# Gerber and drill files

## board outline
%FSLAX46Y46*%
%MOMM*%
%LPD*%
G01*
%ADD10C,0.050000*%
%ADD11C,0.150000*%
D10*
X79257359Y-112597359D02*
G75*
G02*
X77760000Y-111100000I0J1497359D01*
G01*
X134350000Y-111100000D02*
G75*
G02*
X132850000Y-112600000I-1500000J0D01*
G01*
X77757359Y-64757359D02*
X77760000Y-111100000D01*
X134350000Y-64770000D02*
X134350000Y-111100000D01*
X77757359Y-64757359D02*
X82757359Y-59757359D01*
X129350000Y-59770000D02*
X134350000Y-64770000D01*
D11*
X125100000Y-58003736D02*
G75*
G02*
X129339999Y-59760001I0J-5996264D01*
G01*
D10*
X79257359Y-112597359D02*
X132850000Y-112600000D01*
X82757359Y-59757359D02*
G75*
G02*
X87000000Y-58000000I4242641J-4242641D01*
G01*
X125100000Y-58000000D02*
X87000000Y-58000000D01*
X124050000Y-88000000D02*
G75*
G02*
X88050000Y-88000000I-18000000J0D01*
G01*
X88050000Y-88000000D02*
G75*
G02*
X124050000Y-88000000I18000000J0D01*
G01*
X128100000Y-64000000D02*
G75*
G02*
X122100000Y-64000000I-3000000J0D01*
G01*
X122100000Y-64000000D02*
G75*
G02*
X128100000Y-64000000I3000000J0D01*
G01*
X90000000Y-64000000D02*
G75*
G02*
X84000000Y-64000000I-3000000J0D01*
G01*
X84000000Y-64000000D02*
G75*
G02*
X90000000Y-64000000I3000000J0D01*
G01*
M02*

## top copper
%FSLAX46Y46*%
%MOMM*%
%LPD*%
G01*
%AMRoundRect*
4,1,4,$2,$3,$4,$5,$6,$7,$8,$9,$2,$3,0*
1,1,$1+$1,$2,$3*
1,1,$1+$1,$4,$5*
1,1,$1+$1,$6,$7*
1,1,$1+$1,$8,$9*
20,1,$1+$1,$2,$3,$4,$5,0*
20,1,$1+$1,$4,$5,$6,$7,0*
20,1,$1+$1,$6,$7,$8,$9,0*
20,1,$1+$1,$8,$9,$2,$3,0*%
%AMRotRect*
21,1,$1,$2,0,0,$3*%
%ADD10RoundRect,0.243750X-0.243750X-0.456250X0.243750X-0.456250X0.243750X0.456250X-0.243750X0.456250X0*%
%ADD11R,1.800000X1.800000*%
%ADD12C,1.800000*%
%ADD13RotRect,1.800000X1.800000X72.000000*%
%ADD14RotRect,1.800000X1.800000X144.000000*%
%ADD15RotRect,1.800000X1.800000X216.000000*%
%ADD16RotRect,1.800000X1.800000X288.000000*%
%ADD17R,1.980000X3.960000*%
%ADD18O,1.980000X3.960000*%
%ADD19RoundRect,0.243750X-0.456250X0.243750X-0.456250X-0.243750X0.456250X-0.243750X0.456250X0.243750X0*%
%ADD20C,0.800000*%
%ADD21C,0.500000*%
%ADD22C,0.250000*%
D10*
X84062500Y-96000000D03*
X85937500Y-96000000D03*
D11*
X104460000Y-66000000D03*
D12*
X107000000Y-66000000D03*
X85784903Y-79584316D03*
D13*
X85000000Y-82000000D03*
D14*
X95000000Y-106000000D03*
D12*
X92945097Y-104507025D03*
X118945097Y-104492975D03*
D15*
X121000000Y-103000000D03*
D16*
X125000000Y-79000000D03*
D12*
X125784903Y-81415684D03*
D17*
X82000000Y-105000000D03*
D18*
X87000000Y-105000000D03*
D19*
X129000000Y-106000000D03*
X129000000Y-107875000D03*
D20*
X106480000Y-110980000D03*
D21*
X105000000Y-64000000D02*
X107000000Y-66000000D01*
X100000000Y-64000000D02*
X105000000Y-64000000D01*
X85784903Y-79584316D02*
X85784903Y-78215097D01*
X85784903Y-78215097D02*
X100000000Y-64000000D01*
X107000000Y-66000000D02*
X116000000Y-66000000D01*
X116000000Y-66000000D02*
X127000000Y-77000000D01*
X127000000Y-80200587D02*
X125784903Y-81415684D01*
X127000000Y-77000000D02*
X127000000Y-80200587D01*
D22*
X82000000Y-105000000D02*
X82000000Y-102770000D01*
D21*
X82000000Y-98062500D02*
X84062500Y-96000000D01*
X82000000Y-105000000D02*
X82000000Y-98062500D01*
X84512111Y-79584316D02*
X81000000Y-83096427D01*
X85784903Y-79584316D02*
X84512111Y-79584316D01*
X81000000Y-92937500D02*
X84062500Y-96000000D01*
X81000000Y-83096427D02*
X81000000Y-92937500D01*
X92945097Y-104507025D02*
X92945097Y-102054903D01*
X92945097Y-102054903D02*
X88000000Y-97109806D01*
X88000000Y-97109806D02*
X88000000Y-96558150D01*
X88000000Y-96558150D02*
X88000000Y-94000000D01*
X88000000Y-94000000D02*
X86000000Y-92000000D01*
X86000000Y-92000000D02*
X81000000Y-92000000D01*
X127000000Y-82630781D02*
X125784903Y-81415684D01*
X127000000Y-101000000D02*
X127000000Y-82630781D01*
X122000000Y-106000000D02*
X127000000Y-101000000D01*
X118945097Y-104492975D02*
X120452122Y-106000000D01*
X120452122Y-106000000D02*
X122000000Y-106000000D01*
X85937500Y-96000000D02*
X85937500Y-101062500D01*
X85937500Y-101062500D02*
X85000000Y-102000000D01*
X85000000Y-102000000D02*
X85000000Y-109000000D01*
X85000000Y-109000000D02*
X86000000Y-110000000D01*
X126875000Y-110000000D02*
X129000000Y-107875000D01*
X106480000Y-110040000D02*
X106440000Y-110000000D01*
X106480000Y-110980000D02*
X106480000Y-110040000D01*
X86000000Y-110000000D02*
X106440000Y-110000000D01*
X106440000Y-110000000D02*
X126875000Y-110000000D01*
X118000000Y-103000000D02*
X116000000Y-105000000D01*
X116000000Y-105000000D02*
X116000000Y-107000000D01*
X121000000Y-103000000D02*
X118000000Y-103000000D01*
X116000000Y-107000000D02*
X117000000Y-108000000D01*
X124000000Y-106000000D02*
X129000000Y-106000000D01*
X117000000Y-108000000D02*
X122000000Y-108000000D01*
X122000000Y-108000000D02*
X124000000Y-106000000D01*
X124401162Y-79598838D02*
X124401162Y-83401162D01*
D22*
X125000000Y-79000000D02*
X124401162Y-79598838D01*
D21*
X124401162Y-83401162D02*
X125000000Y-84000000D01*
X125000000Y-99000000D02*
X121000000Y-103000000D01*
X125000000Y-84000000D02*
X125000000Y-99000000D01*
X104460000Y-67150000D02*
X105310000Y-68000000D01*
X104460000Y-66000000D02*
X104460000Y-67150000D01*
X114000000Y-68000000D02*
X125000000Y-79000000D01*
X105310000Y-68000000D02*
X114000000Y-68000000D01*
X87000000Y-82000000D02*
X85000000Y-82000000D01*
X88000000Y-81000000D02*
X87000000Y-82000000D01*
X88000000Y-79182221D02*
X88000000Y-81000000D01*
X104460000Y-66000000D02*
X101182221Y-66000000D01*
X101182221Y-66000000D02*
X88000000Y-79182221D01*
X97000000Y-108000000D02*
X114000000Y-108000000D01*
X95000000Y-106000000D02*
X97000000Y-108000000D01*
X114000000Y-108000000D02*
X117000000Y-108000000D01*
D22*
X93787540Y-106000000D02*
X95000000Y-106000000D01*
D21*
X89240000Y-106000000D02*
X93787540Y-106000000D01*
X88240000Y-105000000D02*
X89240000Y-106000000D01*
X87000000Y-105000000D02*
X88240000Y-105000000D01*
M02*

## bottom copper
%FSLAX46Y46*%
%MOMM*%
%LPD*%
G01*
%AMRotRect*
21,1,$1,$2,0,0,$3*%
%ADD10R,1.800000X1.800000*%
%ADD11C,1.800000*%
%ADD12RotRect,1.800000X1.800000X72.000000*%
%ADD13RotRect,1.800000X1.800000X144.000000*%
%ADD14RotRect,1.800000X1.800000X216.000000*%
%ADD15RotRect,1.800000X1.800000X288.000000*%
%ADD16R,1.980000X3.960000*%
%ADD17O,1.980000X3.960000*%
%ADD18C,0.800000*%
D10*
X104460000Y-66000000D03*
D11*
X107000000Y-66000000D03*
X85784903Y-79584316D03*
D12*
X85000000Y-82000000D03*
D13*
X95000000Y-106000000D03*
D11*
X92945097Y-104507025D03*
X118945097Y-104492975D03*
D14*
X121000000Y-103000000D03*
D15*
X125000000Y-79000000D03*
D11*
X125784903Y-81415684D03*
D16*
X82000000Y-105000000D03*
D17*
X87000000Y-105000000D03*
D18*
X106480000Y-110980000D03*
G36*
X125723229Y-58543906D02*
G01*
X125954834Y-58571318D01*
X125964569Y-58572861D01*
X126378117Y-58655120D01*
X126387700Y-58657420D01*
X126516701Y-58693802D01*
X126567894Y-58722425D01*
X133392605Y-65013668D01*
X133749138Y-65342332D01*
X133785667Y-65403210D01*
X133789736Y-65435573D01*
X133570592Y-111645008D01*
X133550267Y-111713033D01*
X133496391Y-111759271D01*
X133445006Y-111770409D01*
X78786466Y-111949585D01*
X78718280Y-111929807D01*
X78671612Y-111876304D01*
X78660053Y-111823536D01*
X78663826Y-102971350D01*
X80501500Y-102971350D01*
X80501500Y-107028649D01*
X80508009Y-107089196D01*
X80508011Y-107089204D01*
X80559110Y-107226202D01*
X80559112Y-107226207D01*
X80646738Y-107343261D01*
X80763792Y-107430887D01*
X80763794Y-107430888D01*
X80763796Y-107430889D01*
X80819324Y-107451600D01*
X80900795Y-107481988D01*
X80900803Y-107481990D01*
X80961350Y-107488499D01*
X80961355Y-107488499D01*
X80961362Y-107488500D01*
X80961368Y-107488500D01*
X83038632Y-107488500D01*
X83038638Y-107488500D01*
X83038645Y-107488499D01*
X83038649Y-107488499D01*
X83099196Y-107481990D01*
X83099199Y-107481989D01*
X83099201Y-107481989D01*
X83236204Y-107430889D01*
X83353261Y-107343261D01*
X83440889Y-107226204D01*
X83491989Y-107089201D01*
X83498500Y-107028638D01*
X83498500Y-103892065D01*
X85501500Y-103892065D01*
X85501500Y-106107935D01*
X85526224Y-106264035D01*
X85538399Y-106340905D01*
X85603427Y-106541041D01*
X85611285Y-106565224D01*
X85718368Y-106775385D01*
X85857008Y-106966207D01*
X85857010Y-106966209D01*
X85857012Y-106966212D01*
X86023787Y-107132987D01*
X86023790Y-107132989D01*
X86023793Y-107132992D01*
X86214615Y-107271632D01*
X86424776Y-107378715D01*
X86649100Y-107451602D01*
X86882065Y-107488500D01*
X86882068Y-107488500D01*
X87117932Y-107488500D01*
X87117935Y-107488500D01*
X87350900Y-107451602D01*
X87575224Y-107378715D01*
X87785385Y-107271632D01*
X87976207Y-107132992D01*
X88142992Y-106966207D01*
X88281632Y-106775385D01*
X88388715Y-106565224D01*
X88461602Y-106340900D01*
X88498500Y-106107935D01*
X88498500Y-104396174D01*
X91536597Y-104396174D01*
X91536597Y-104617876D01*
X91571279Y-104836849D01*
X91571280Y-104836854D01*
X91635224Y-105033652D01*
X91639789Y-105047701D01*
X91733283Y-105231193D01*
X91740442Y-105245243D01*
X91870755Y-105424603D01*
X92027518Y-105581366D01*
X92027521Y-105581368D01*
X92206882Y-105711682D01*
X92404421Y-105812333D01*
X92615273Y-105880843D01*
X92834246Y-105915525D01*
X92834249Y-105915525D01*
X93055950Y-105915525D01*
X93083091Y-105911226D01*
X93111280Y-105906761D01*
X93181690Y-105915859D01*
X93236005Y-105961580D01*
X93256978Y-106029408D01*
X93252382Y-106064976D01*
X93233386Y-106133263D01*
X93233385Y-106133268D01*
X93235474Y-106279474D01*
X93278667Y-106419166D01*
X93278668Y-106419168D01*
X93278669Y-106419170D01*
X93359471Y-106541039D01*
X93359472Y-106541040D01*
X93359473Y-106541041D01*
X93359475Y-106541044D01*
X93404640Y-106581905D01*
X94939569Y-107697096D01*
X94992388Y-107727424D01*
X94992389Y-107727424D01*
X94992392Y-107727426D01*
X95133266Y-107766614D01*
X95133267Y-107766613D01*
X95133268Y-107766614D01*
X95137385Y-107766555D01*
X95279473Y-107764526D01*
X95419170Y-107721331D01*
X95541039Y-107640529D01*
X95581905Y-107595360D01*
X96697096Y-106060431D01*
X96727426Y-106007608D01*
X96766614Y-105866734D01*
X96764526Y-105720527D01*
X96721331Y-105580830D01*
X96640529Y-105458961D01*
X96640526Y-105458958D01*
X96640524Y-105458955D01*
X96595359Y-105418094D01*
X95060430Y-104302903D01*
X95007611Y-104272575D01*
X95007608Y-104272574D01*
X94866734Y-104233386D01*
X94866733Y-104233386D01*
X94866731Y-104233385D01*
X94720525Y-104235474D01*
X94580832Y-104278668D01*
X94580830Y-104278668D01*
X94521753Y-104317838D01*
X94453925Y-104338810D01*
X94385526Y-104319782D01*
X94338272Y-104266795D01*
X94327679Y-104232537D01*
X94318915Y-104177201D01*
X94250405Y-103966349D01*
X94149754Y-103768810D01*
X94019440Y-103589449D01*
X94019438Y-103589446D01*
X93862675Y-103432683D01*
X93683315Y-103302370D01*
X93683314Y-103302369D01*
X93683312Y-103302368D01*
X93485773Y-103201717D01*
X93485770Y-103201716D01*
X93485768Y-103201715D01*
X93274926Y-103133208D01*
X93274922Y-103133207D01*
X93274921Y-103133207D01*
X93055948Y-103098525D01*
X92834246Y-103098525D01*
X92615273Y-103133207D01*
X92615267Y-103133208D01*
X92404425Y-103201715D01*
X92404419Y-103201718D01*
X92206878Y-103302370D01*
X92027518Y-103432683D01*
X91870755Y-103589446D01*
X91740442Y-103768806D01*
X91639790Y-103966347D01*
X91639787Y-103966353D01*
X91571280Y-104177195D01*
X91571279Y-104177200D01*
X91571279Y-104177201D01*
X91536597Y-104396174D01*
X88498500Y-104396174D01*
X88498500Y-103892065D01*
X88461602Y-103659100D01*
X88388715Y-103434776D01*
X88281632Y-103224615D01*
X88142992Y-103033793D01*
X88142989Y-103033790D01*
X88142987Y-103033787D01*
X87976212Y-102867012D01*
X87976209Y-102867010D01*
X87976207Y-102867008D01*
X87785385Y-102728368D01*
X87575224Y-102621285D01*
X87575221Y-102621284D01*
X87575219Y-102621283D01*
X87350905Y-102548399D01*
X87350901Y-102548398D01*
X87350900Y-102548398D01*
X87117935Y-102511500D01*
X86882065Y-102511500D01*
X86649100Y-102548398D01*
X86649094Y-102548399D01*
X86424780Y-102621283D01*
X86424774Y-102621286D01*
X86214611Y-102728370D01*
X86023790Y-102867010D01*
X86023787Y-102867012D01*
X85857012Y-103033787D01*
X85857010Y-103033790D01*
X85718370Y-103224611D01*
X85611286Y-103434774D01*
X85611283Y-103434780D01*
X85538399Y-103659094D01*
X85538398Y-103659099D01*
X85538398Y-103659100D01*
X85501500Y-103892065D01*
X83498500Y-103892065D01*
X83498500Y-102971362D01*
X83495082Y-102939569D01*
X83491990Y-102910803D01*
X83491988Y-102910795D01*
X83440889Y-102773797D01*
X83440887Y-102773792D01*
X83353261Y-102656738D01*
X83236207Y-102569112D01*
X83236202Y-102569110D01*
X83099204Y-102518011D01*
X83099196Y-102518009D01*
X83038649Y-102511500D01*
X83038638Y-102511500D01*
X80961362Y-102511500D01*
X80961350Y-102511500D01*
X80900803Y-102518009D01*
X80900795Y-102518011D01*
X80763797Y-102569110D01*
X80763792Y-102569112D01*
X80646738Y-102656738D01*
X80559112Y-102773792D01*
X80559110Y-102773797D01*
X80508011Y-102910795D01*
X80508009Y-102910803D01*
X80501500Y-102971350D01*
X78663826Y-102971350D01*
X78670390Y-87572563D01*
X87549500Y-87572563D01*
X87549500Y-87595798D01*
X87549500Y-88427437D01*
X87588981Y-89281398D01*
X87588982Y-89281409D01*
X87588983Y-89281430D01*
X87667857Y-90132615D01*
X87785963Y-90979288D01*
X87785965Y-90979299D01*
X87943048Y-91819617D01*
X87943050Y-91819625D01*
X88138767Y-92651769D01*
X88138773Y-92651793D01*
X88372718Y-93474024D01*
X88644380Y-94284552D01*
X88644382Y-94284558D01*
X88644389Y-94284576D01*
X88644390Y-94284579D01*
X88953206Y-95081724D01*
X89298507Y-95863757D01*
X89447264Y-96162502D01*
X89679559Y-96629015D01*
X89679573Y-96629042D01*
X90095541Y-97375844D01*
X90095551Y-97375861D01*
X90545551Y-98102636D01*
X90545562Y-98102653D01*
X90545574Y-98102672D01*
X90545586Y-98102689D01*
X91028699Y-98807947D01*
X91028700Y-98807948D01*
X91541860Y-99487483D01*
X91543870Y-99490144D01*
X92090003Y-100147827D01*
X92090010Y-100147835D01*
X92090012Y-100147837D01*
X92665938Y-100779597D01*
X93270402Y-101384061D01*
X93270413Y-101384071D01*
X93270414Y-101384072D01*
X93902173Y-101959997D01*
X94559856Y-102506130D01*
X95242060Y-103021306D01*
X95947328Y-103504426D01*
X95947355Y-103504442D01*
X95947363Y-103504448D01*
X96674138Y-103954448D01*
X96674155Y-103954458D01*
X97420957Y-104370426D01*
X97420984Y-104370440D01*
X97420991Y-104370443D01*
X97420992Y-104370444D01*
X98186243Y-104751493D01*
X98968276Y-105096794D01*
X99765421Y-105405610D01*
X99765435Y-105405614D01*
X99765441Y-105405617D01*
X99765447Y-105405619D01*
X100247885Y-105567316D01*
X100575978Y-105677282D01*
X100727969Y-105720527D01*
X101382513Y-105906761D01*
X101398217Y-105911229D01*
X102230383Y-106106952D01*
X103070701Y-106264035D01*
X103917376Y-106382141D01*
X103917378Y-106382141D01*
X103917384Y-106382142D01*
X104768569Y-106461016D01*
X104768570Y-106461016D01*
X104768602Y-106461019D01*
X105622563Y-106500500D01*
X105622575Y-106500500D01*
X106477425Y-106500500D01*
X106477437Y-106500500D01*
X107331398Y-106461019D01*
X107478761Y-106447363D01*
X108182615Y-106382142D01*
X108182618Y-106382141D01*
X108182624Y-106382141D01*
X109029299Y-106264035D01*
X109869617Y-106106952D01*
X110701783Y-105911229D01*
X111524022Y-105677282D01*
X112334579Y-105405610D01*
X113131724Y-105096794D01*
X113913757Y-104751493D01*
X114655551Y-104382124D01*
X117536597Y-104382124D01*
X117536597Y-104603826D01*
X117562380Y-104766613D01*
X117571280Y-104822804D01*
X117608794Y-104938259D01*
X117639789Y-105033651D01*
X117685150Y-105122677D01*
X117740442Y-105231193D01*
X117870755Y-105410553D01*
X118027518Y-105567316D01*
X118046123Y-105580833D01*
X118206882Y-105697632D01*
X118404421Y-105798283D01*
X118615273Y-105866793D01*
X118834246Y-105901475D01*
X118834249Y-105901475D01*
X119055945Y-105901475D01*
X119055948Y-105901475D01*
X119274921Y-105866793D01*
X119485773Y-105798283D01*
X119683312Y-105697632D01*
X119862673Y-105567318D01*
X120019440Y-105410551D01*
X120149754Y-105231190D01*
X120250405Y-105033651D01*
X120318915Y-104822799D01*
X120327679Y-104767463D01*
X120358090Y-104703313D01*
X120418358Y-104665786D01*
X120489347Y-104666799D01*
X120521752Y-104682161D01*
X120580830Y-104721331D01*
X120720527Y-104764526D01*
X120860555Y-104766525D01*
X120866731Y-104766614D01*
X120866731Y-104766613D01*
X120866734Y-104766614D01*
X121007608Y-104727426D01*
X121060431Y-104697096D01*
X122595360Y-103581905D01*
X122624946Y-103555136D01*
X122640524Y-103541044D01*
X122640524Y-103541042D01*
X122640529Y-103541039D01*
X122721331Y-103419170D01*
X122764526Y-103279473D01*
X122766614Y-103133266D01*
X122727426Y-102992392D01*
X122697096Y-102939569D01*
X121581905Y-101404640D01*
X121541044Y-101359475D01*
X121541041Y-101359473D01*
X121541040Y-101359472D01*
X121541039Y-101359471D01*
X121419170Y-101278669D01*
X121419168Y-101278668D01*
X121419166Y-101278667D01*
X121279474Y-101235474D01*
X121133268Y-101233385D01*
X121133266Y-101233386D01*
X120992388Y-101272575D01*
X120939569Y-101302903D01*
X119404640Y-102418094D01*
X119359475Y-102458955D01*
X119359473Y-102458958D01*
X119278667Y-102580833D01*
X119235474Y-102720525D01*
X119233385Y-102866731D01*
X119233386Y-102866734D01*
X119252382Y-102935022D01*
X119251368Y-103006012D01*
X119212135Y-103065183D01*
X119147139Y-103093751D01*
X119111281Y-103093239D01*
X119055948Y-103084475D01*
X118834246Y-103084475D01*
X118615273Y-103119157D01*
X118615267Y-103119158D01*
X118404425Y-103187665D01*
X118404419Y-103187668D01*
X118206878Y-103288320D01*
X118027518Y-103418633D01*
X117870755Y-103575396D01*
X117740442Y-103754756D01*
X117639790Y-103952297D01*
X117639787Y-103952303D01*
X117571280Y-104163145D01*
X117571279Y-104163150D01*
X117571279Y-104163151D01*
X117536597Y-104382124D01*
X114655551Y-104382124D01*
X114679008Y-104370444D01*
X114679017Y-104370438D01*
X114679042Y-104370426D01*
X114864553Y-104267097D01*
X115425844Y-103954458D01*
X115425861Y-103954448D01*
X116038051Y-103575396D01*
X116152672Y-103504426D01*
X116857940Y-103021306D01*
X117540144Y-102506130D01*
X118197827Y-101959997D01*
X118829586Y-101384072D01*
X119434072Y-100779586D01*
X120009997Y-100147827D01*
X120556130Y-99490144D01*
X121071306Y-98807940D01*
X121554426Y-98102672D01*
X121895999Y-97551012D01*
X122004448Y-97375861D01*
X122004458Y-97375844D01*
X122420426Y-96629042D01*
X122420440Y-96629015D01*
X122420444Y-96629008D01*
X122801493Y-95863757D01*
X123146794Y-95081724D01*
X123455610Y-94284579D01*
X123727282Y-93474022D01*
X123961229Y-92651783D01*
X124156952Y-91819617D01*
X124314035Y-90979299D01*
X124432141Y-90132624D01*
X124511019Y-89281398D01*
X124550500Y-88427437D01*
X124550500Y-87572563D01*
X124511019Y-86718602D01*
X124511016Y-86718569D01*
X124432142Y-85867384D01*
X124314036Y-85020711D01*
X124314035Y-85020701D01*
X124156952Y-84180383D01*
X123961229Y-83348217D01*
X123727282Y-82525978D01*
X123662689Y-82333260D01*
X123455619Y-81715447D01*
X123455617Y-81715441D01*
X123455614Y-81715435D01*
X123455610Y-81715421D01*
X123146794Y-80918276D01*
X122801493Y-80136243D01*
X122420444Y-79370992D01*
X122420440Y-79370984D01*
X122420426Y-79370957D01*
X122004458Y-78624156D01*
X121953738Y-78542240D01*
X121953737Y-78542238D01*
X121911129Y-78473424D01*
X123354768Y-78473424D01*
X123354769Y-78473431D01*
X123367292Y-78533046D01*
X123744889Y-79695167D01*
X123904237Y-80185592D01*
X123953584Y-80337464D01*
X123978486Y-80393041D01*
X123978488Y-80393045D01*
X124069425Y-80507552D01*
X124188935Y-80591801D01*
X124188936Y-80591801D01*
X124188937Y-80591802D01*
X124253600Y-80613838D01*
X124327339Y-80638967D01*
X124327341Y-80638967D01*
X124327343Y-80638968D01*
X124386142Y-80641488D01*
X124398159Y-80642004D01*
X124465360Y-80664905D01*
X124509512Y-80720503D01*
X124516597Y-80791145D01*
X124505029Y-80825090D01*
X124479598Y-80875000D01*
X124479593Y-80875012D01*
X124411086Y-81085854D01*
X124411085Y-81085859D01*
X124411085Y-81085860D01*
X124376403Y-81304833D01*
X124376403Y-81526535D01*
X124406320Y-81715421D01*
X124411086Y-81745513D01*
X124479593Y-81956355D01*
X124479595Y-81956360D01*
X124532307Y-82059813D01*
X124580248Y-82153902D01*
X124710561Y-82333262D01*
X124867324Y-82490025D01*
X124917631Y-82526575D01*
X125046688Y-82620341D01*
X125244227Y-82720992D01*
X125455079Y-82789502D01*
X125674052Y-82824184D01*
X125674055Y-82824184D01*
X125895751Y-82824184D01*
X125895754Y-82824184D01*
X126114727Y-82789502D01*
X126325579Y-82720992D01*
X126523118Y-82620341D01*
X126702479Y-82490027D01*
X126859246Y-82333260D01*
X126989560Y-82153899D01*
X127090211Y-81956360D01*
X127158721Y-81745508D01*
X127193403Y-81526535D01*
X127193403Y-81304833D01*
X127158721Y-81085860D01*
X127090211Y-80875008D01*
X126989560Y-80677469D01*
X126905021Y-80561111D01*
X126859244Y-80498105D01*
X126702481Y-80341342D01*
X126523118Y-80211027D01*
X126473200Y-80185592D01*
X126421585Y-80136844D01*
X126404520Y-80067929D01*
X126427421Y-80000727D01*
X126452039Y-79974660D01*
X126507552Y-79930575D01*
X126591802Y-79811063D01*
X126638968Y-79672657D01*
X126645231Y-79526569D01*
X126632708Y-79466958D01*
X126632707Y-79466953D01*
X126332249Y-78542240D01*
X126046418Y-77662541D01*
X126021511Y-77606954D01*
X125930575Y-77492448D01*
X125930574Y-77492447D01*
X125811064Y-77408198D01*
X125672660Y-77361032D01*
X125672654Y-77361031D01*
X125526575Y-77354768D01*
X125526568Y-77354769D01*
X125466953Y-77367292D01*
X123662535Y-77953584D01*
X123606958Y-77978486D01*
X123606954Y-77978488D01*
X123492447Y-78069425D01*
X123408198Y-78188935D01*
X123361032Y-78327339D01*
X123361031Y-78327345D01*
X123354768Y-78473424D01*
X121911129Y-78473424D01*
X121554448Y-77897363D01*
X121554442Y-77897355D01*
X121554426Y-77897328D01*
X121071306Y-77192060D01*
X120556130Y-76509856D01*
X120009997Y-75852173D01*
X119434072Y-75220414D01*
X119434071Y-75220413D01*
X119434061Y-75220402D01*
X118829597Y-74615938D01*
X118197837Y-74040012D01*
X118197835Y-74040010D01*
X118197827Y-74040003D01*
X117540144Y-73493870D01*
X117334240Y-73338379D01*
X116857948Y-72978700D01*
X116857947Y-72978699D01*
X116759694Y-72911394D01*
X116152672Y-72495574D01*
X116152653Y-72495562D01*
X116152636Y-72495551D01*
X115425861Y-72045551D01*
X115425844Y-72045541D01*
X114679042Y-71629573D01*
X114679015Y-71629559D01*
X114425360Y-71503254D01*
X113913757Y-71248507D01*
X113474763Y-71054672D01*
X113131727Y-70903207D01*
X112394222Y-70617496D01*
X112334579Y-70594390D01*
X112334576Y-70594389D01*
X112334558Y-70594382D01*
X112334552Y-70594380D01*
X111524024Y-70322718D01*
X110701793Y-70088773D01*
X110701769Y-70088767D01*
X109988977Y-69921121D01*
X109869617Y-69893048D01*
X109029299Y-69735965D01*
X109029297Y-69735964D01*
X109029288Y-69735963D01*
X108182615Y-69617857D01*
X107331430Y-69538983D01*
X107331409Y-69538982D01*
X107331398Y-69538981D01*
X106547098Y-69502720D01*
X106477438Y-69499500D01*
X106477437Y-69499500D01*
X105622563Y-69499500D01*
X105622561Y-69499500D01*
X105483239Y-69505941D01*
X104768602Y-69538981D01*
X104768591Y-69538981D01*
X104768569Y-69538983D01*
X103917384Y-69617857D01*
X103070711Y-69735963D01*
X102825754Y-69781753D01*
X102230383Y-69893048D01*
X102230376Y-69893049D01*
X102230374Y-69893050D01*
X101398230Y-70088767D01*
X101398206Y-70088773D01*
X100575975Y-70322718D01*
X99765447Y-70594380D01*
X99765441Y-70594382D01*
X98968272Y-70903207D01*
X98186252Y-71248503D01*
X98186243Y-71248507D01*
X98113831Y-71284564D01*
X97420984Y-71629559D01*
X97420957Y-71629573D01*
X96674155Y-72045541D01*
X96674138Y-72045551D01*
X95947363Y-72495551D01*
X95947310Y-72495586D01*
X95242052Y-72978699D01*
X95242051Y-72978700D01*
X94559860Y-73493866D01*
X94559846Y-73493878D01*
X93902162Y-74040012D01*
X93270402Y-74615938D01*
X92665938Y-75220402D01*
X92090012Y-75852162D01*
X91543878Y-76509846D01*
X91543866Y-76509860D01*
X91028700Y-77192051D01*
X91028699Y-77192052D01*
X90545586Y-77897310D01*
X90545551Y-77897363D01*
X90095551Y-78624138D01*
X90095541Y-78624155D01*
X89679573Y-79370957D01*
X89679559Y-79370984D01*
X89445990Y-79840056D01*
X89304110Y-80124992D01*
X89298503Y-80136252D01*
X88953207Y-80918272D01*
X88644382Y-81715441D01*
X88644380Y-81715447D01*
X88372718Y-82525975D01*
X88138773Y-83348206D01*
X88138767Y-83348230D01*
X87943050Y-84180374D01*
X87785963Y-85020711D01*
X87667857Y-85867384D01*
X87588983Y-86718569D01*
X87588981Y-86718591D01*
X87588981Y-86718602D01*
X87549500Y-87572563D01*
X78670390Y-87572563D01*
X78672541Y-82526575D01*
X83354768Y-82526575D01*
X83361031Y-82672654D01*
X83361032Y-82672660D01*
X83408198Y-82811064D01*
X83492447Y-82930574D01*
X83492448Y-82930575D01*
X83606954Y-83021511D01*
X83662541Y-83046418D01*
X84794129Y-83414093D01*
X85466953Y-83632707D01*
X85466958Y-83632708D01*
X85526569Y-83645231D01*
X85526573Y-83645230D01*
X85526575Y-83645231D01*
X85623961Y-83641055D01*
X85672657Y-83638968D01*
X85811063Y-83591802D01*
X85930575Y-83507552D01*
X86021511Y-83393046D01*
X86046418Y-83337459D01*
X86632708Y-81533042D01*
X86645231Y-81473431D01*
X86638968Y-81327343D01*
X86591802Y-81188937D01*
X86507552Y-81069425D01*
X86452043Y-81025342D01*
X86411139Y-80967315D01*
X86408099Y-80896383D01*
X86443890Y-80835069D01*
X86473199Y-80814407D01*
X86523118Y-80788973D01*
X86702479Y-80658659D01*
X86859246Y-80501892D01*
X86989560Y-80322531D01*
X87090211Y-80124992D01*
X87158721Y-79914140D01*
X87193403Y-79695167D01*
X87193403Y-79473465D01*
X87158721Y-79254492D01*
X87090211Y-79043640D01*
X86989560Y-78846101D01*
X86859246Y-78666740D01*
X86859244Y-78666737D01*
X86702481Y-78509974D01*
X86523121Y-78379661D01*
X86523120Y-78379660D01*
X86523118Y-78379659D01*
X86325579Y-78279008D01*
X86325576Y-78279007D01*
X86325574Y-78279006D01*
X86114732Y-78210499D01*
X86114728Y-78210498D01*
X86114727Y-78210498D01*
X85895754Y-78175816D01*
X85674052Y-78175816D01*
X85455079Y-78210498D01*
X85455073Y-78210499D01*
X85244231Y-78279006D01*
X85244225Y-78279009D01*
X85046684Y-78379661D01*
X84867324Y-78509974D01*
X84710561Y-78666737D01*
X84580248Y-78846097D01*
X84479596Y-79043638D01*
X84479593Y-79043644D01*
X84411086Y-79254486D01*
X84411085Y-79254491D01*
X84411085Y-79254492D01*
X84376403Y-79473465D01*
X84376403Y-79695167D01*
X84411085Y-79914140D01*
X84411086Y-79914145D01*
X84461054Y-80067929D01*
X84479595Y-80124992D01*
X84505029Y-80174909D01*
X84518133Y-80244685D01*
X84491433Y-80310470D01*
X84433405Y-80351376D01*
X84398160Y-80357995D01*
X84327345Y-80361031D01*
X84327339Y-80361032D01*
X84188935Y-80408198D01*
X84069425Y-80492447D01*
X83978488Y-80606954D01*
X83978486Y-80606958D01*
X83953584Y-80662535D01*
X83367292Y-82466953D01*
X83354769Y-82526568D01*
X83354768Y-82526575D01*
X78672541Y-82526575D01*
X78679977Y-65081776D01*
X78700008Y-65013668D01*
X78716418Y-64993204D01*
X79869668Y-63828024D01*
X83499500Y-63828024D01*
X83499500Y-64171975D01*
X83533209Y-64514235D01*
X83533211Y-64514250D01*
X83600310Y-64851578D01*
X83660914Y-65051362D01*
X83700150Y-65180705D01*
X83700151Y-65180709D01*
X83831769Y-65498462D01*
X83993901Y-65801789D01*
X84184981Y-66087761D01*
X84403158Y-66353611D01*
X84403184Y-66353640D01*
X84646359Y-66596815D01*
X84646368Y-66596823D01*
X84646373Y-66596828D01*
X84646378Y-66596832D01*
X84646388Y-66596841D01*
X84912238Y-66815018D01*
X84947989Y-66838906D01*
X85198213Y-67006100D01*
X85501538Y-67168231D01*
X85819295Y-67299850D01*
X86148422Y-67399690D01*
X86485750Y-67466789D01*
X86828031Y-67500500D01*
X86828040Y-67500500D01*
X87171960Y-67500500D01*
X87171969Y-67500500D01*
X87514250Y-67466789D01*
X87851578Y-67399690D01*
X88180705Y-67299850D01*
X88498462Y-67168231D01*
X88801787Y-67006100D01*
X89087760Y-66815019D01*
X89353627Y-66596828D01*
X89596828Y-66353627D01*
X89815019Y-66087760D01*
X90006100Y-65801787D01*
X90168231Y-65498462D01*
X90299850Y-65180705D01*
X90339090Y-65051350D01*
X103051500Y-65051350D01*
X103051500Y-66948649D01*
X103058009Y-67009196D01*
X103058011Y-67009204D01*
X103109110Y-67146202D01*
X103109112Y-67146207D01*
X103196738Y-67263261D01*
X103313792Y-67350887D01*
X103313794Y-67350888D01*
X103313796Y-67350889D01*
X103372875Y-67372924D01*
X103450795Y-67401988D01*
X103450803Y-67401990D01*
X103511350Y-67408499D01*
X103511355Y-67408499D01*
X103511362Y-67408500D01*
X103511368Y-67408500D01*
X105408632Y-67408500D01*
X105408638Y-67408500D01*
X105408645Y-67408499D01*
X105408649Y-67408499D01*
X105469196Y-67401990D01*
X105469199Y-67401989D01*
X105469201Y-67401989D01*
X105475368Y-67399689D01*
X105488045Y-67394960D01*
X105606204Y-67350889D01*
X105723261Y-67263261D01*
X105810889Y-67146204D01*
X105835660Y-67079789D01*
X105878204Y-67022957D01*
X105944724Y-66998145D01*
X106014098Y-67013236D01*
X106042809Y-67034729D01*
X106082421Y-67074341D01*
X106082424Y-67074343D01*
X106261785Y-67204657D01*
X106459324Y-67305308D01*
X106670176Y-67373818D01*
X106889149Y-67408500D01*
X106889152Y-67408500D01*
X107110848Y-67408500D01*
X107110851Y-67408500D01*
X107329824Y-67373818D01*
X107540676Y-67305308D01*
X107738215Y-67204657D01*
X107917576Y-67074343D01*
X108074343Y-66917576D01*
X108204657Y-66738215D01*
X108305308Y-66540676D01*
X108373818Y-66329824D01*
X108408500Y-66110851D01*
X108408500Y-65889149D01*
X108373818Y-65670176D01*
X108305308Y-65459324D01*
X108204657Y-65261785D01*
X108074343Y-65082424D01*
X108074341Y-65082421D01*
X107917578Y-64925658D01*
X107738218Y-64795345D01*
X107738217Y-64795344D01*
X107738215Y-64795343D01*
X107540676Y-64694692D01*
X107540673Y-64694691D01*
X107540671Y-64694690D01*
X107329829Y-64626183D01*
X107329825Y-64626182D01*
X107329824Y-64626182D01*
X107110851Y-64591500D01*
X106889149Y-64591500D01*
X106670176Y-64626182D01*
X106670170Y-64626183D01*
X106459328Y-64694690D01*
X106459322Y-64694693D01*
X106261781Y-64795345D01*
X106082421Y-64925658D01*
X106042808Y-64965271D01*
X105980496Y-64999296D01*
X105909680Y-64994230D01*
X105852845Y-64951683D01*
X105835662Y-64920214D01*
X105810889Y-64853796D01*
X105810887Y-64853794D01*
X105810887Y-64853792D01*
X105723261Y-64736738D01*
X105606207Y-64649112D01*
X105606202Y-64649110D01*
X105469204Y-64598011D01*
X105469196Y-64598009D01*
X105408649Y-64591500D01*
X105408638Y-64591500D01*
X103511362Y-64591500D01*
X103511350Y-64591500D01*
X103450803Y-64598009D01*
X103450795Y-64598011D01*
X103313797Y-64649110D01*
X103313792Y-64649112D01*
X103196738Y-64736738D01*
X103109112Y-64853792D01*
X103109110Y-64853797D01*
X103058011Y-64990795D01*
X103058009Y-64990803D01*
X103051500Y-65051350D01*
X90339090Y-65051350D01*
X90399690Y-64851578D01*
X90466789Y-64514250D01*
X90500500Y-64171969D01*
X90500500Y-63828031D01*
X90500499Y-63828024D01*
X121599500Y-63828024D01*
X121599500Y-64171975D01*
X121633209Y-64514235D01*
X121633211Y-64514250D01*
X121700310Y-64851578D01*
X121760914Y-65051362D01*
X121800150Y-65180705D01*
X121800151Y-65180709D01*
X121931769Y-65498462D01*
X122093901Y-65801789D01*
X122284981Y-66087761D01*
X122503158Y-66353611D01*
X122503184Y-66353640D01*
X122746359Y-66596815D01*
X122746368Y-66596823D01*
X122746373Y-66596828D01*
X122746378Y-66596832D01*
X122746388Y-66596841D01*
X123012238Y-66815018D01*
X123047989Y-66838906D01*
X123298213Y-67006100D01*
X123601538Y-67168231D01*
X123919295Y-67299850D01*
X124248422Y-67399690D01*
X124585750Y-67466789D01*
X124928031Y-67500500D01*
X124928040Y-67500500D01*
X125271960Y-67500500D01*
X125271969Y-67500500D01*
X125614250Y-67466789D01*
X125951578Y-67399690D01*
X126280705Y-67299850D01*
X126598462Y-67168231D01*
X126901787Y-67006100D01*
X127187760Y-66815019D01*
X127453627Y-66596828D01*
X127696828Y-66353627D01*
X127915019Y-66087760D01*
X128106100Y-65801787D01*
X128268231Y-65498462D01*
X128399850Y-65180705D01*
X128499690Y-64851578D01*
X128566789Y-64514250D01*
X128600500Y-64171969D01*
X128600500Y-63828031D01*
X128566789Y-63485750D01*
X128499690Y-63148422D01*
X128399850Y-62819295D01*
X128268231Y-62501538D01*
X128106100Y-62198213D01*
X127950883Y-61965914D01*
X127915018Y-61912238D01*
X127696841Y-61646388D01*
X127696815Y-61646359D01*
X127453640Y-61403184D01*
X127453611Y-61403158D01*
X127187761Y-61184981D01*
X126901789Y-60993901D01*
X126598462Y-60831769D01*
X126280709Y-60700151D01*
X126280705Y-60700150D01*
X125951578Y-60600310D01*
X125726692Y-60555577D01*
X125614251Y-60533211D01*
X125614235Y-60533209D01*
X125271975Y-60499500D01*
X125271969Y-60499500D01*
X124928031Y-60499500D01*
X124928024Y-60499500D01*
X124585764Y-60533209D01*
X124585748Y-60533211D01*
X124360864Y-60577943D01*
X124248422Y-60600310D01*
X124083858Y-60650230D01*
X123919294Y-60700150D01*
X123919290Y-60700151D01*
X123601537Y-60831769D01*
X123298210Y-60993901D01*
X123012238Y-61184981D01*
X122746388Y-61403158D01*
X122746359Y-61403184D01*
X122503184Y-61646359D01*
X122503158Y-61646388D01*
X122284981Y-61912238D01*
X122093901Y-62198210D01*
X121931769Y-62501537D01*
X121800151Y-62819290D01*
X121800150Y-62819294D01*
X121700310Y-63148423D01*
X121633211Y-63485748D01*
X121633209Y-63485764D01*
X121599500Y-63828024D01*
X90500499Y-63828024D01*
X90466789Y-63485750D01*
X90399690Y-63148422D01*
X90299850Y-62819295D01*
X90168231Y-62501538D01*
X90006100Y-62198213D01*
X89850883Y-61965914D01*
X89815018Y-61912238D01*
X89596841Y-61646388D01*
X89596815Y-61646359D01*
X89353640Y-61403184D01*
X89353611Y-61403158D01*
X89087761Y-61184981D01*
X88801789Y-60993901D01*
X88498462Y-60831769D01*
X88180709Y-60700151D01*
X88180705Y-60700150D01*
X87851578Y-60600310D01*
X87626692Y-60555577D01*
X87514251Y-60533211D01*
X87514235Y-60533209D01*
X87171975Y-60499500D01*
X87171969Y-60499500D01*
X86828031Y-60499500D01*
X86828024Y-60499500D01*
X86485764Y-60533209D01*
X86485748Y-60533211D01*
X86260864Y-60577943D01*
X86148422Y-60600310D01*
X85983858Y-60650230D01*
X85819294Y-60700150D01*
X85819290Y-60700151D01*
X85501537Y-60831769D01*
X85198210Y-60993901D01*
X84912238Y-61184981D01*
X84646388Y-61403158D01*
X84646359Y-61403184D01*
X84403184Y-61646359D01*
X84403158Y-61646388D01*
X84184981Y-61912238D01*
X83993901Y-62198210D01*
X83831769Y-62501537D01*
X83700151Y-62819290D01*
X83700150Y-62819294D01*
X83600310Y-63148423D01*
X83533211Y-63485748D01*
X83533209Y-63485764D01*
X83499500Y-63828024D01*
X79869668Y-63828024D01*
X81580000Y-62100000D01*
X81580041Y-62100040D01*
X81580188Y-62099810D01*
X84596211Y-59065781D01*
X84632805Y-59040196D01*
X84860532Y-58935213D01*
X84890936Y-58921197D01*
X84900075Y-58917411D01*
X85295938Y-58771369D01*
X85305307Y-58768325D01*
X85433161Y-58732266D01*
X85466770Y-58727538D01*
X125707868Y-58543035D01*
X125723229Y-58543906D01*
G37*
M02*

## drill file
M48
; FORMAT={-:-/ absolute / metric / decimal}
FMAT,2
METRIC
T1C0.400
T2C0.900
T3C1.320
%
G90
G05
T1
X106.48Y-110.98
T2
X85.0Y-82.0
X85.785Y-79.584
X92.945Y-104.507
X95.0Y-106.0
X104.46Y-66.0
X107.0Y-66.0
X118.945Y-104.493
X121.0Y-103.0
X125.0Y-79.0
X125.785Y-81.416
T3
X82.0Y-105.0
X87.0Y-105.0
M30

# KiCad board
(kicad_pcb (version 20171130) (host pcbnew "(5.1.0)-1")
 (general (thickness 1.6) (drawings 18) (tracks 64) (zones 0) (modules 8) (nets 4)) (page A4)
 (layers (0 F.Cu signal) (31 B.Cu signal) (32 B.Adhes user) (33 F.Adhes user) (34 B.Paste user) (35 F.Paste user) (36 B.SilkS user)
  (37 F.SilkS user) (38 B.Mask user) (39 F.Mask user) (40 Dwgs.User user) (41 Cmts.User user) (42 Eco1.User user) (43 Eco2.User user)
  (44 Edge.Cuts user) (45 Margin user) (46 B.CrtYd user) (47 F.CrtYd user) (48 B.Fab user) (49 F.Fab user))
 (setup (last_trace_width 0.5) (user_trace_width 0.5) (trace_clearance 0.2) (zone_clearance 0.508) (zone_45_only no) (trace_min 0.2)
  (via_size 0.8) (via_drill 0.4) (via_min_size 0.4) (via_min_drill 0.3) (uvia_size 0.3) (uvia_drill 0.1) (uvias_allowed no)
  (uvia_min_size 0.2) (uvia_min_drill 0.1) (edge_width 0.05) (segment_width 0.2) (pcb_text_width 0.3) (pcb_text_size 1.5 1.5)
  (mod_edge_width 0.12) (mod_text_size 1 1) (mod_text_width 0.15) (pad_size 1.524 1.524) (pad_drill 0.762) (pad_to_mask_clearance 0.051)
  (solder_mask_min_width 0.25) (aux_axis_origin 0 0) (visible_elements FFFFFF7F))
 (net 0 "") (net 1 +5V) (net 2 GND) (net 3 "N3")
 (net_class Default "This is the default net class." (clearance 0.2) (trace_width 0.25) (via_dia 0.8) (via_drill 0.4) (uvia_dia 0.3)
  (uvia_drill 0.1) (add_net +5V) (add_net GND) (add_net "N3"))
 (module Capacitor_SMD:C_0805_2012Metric (layer F.Cu) (at 85 96)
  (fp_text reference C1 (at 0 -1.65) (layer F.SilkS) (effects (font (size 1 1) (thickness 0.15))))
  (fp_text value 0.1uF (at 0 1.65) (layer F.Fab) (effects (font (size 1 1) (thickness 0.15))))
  (pad 1 smd roundrect (at -0.9375 0) (size 0.975 1.4) (layers F.Cu F.Paste F.Mask) (roundrect_rratio 0.25) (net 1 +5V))
  (pad 2 smd roundrect (at 0.9375 0) (size 0.975 1.4) (layers F.Cu F.Paste F.Mask) (roundrect_rratio 0.25) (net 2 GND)))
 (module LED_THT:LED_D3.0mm (layer F.Cu) (at 104.46 66)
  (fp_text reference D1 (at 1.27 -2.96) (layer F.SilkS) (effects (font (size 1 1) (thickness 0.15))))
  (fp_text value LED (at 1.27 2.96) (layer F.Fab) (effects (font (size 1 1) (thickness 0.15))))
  (pad 1 thru_hole rect (at 0 0) (size 1.8 1.8) (drill 0.9) (layers *.Cu *.Mask) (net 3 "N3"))
  (pad 2 thru_hole circle (at 2.54 0) (size 1.8 1.8) (drill 0.9) (layers *.Cu *.Mask) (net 1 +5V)))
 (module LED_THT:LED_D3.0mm (layer F.Cu) (at 85 82 72)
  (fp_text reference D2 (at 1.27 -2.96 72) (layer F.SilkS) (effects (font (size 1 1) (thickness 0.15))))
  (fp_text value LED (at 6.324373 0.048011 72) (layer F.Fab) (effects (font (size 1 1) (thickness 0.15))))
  (pad 2 thru_hole circle (at 2.54 0 72) (size 1.8 1.8) (drill 0.9) (layers *.Cu *.Mask) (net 1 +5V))
  (pad 1 thru_hole rect (at 0 0 72) (size 1.8 1.8) (drill 0.9) (layers *.Cu *.Mask) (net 3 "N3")))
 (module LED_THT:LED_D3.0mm (layer F.Cu) (at 95 106 144)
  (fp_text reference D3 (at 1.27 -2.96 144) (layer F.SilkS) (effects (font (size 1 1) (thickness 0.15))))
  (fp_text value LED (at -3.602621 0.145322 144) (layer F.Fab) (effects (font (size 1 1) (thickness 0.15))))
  (pad 1 thru_hole rect (at 0 0 144) (size 1.8 1.8) (drill 0.9) (layers *.Cu *.Mask) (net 3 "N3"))
  (pad 2 thru_hole circle (at 2.54 0 144) (size 1.8 1.8) (drill 0.9) (layers *.Cu *.Mask) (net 1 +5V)))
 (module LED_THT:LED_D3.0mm (layer F.Cu) (at 121 103 216)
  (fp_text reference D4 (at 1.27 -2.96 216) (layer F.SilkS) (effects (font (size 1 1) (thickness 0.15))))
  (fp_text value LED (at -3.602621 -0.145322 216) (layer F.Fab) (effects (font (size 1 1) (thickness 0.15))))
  (pad 2 thru_hole circle (at 2.54 0 216) (size 1.8 1.8) (drill 0.9) (layers *.Cu *.Mask) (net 1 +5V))
  (pad 1 thru_hole rect (at 0 0 216) (size 1.8 1.8) (drill 0.9) (layers *.Cu *.Mask) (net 3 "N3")))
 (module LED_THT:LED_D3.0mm (layer F.Cu) (at 125 79 288)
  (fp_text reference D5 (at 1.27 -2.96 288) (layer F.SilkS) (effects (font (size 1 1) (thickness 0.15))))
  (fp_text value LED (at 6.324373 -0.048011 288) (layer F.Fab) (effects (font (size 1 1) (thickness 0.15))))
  (pad 1 thru_hole rect (at 0 0 288) (size 1.8 1.8) (drill 0.9) (layers *.Cu *.Mask) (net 3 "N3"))
  (pad 2 thru_hole circle (at 2.54 0 288) (size 1.8 1.8) (drill 0.9) (layers *.Cu *.Mask) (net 1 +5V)))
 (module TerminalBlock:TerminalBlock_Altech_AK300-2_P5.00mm (layer F.Cu) (at 82 105)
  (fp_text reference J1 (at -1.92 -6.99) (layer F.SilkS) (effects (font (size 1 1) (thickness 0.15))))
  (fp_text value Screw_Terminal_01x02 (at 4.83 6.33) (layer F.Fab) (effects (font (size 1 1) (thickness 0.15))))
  (pad 1 thru_hole rect (at 0 0) (size 1.98 3.96) (drill 1.32) (layers *.Cu *.Mask) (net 1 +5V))
  (pad 2 thru_hole oval (at 5 0) (size 1.98 3.96) (drill 1.32) (layers *.Cu *.Mask) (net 3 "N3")))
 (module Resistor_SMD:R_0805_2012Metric (layer F.Cu) (at 129 106.9375 270)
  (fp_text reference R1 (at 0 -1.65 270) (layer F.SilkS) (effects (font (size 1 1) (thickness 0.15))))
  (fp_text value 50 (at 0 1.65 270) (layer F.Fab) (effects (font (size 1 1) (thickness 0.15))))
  (pad 1 smd roundrect (at -0.9375 0 270) (size 0.975 1.4) (layers F.Cu F.Paste F.Mask) (roundrect_rratio 0.25) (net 3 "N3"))
  (pad 2 smd roundrect (at 0.9375 0 270) (size 0.975 1.4) (layers F.Cu F.Paste F.Mask) (roundrect_rratio 0.25) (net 2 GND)))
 (gr_arc (start 79.257359 111.1) (end 77.76 111.1) (angle -90) (layer Edge.Cuts) (width 0.05))
 (gr_arc (start 132.85 111.1) (end 132.85 112.6) (angle -90) (layer Edge.Cuts) (width 0.05))
 (gr_line (start 77.757359 64.757359) (end 77.76 111.1) (layer Edge.Cuts) (width 0.05))
 (gr_line (start 134.35 64.77) (end 134.35 111.1) (layer Edge.Cuts) (width 0.05))
 (gr_line (start 77.757359 64.757359) (end 82.757359 59.757359) (layer Edge.Cuts) (width 0.05))
 (gr_line (start 129.35 59.77) (end 134.35 64.77) (layer Edge.Cuts) (width 0.05))
 (gr_arc (start 125.1 64) (end 129.339999 59.760001) (angle -45) (layer Edge.Cuts) (width 0.15))
 (gr_line (start 79.257359 112.597359) (end 132.85 112.6) (layer Edge.Cuts) (width 0.05))
 (gr_arc (start 87 64) (end 87 58) (angle -45) (layer Edge.Cuts) (width 0.05))
 (gr_line (start 125.1 58) (end 87 58) (layer Edge.Cuts) (width 0.05))
 (gr_circle (center 106.05 88) (end 124.05 88) (layer Edge.Cuts) (width 0.05))
 (gr_circle (center 125.1 64) (end 128.1 64) (layer Edge.Cuts) (width 0.05))
 (gr_circle (center 87 64) (end 90 64) (layer Edge.Cuts) (width 0.05))
 (via (at 106.48 110.98) (size 0.8) (drill 0.4) (layers F.Cu B.Cu) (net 2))
 (segment (start 105 64) (end 107 66) (width 0.5) (layer F.Cu) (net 1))
 (segment (start 100 64) (end 105 64) (width 0.5) (layer F.Cu) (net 1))
 (segment (start 85.784903 79.584316) (end 85.784903 78.215097) (width 0.5) (layer F.Cu) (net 1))
 (segment (start 85.784903 78.215097) (end 100 64) (width 0.5) (layer F.Cu) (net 1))
 (segment (start 107 66) (end 116 66) (width 0.5) (layer F.Cu) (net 1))
 (segment (start 116 66) (end 127 77) (width 0.5) (layer F.Cu) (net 1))
 (segment (start 127 80.200587) (end 125.784903 81.415684) (width 0.5) (layer F.Cu) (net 1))
 (segment (start 127 77) (end 127 80.200587) (width 0.5) (layer F.Cu) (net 1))
 (segment (start 82 105) (end 82 102.77) (width 0.25) (layer F.Cu) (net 1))
 (segment (start 82 98.0625) (end 84.0625 96) (width 0.5) (layer F.Cu) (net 1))
 (segment (start 82 105) (end 82 98.0625) (width 0.5) (layer F.Cu) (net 1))
 (segment (start 84.512111 79.584316) (end 81 83.096427) (width 0.5) (layer F.Cu) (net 1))
 (segment (start 85.784903 79.584316) (end 84.512111 79.584316) (width 0.5) (layer F.Cu) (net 1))
 (segment (start 81 92.9375) (end 84.0625 96) (width 0.5) (layer F.Cu) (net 1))
 (segment (start 81 83.096427) (end 81 92.9375) (width 0.5) (layer F.Cu) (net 1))
 (segment (start 92.945097 104.507025) (end 92.945097 102.054903) (width 0.5) (layer F.Cu) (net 1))
 (segment (start 92.945097 102.054903) (end 88 97.109806) (width 0.5) (layer F.Cu) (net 1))
 (segment (start 88 97.109806) (end 88 96.55815) (width 0.5) (layer F.Cu) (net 1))
 (segment (start 88 96.55815) (end 88 94) (width 0.5) (layer F.Cu) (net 1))
 (segment (start 88 94) (end 86 92) (width 0.5) (layer F.Cu) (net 1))
 (segment (start 86 92) (end 81 92) (width 0.5) (layer F.Cu) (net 1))
 (segment (start 127 82.630781) (end 125.784903 81.415684) (width 0.5) (layer F.Cu) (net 1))
 (segment (start 127 101) (end 127 82.630781) (width 0.5) (layer F.Cu) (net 1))
 (segment (start 122 106) (end 127 101) (width 0.5) (layer F.Cu) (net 1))
 (segment (start 118.945097 104.492975) (end 120.452122 106) (width 0.5) (layer F.Cu) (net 1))
 (segment (start 120.452122 106) (end 122 106) (width 0.5) (layer F.Cu) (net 1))
 (segment (start 85.9375 96) (end 85.9375 101.0625) (width 0.5) (layer F.Cu) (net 2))
 (segment (start 85.9375 101.0625) (end 85 102) (width 0.5) (layer F.Cu) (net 2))
 (segment (start 85 102) (end 85 109) (width 0.5) (layer F.Cu) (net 2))
 (segment (start 85 109) (end 86 110) (width 0.5) (layer F.Cu) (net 2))
 (segment (start 126.875 110) (end 129 107.875) (width 0.5) (layer F.Cu) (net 2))
 (segment (start 106.48 110.04) (end 106.44 110) (width 0.5) (layer F.Cu) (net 2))
 (segment (start 106.48 110.98) (end 106.48 110.04) (width 0.5) (layer F.Cu) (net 2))
 (segment (start 86 110) (end 106.44 110) (width 0.5) (layer F.Cu) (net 2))
 (segment (start 106.44 110) (end 126.875 110) (width 0.5) (layer F.Cu) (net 2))
 (segment (start 118 103) (end 116 105) (width 0.5) (layer F.Cu) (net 3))
 (segment (start 116 105) (end 116 107) (width 0.5) (layer F.Cu) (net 3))
 (segment (start 121 103) (end 118 103) (width 0.5) (layer F.Cu) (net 3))
 (segment (start 116 107) (end 117 108) (width 0.5) (layer F.Cu) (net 3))
 (segment (start 124 106) (end 129 106) (width 0.5) (layer F.Cu) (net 3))
 (segment (start 117 108) (end 122 108) (width 0.5) (layer F.Cu) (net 3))
 (segment (start 122 108) (end 124 106) (width 0.5) (layer F.Cu) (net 3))
 (segment (start 124.401162 79.598838) (end 124.401162 83.401162) (width 0.5) (layer F.Cu) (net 3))
 (segment (start 125 79) (end 124.401162 79.598838) (width 0.25) (layer F.Cu) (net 3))
 (segment (start 124.401162 83.401162) (end 125 84) (width 0.5) (layer F.Cu) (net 3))
 (segment (start 125 99) (end 121 103) (width 0.5) (layer F.Cu) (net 3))
 (segment (start 125 84) (end 125 99) (width 0.5) (layer F.Cu) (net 3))
 (segment (start 104.46 67.15) (end 105.31 68) (width 0.5) (layer F.Cu) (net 3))
 (segment (start 104.46 66) (end 104.46 67.15) (width 0.5) (layer F.Cu) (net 3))
 (segment (start 114 68) (end 125 79) (width 0.5) (layer F.Cu) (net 3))
 (segment (start 105.31 68) (end 114 68) (width 0.5) (layer F.Cu) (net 3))
 (segment (start 87 82) (end 85 82) (width 0.5) (layer F.Cu) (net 3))
 (segment (start 88 81) (end 87 82) (width 0.5) (layer F.Cu) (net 3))
 (segment (start 88 79.182221) (end 88 81) (width 0.5) (layer F.Cu) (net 3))
 (segment (start 104.46 66) (end 101.182221 66) (width 0.5) (layer F.Cu) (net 3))
 (segment (start 101.182221 66) (end 88 79.182221) (width 0.5) (layer F.Cu) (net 3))
 (segment (start 97 108) (end 114 108) (width 0.5) (layer F.Cu) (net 3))
 (segment (start 95 106) (end 97 108) (width 0.5) (layer F.Cu) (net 3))
 (segment (start 114 108) (end 117 108) (width 0.5) (layer F.Cu) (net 3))
 (segment (start 93.78754 106) (end 95 106) (width 0.25) (layer F.Cu) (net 3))
 (segment (start 89.24 106) (end 93.78754 106) (width 0.5) (layer F.Cu) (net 3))
 (segment (start 88.24 105) (end 89.24 106) (width 0.5) (layer F.Cu) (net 3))
 (segment (start 87 105) (end 88.24 105) (width 0.5) (layer F.Cu) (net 3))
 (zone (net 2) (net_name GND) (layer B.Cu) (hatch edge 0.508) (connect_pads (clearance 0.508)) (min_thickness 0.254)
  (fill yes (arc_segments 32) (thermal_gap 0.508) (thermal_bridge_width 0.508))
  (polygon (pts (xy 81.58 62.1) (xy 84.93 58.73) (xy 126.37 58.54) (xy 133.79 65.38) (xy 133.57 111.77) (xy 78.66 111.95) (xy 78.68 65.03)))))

